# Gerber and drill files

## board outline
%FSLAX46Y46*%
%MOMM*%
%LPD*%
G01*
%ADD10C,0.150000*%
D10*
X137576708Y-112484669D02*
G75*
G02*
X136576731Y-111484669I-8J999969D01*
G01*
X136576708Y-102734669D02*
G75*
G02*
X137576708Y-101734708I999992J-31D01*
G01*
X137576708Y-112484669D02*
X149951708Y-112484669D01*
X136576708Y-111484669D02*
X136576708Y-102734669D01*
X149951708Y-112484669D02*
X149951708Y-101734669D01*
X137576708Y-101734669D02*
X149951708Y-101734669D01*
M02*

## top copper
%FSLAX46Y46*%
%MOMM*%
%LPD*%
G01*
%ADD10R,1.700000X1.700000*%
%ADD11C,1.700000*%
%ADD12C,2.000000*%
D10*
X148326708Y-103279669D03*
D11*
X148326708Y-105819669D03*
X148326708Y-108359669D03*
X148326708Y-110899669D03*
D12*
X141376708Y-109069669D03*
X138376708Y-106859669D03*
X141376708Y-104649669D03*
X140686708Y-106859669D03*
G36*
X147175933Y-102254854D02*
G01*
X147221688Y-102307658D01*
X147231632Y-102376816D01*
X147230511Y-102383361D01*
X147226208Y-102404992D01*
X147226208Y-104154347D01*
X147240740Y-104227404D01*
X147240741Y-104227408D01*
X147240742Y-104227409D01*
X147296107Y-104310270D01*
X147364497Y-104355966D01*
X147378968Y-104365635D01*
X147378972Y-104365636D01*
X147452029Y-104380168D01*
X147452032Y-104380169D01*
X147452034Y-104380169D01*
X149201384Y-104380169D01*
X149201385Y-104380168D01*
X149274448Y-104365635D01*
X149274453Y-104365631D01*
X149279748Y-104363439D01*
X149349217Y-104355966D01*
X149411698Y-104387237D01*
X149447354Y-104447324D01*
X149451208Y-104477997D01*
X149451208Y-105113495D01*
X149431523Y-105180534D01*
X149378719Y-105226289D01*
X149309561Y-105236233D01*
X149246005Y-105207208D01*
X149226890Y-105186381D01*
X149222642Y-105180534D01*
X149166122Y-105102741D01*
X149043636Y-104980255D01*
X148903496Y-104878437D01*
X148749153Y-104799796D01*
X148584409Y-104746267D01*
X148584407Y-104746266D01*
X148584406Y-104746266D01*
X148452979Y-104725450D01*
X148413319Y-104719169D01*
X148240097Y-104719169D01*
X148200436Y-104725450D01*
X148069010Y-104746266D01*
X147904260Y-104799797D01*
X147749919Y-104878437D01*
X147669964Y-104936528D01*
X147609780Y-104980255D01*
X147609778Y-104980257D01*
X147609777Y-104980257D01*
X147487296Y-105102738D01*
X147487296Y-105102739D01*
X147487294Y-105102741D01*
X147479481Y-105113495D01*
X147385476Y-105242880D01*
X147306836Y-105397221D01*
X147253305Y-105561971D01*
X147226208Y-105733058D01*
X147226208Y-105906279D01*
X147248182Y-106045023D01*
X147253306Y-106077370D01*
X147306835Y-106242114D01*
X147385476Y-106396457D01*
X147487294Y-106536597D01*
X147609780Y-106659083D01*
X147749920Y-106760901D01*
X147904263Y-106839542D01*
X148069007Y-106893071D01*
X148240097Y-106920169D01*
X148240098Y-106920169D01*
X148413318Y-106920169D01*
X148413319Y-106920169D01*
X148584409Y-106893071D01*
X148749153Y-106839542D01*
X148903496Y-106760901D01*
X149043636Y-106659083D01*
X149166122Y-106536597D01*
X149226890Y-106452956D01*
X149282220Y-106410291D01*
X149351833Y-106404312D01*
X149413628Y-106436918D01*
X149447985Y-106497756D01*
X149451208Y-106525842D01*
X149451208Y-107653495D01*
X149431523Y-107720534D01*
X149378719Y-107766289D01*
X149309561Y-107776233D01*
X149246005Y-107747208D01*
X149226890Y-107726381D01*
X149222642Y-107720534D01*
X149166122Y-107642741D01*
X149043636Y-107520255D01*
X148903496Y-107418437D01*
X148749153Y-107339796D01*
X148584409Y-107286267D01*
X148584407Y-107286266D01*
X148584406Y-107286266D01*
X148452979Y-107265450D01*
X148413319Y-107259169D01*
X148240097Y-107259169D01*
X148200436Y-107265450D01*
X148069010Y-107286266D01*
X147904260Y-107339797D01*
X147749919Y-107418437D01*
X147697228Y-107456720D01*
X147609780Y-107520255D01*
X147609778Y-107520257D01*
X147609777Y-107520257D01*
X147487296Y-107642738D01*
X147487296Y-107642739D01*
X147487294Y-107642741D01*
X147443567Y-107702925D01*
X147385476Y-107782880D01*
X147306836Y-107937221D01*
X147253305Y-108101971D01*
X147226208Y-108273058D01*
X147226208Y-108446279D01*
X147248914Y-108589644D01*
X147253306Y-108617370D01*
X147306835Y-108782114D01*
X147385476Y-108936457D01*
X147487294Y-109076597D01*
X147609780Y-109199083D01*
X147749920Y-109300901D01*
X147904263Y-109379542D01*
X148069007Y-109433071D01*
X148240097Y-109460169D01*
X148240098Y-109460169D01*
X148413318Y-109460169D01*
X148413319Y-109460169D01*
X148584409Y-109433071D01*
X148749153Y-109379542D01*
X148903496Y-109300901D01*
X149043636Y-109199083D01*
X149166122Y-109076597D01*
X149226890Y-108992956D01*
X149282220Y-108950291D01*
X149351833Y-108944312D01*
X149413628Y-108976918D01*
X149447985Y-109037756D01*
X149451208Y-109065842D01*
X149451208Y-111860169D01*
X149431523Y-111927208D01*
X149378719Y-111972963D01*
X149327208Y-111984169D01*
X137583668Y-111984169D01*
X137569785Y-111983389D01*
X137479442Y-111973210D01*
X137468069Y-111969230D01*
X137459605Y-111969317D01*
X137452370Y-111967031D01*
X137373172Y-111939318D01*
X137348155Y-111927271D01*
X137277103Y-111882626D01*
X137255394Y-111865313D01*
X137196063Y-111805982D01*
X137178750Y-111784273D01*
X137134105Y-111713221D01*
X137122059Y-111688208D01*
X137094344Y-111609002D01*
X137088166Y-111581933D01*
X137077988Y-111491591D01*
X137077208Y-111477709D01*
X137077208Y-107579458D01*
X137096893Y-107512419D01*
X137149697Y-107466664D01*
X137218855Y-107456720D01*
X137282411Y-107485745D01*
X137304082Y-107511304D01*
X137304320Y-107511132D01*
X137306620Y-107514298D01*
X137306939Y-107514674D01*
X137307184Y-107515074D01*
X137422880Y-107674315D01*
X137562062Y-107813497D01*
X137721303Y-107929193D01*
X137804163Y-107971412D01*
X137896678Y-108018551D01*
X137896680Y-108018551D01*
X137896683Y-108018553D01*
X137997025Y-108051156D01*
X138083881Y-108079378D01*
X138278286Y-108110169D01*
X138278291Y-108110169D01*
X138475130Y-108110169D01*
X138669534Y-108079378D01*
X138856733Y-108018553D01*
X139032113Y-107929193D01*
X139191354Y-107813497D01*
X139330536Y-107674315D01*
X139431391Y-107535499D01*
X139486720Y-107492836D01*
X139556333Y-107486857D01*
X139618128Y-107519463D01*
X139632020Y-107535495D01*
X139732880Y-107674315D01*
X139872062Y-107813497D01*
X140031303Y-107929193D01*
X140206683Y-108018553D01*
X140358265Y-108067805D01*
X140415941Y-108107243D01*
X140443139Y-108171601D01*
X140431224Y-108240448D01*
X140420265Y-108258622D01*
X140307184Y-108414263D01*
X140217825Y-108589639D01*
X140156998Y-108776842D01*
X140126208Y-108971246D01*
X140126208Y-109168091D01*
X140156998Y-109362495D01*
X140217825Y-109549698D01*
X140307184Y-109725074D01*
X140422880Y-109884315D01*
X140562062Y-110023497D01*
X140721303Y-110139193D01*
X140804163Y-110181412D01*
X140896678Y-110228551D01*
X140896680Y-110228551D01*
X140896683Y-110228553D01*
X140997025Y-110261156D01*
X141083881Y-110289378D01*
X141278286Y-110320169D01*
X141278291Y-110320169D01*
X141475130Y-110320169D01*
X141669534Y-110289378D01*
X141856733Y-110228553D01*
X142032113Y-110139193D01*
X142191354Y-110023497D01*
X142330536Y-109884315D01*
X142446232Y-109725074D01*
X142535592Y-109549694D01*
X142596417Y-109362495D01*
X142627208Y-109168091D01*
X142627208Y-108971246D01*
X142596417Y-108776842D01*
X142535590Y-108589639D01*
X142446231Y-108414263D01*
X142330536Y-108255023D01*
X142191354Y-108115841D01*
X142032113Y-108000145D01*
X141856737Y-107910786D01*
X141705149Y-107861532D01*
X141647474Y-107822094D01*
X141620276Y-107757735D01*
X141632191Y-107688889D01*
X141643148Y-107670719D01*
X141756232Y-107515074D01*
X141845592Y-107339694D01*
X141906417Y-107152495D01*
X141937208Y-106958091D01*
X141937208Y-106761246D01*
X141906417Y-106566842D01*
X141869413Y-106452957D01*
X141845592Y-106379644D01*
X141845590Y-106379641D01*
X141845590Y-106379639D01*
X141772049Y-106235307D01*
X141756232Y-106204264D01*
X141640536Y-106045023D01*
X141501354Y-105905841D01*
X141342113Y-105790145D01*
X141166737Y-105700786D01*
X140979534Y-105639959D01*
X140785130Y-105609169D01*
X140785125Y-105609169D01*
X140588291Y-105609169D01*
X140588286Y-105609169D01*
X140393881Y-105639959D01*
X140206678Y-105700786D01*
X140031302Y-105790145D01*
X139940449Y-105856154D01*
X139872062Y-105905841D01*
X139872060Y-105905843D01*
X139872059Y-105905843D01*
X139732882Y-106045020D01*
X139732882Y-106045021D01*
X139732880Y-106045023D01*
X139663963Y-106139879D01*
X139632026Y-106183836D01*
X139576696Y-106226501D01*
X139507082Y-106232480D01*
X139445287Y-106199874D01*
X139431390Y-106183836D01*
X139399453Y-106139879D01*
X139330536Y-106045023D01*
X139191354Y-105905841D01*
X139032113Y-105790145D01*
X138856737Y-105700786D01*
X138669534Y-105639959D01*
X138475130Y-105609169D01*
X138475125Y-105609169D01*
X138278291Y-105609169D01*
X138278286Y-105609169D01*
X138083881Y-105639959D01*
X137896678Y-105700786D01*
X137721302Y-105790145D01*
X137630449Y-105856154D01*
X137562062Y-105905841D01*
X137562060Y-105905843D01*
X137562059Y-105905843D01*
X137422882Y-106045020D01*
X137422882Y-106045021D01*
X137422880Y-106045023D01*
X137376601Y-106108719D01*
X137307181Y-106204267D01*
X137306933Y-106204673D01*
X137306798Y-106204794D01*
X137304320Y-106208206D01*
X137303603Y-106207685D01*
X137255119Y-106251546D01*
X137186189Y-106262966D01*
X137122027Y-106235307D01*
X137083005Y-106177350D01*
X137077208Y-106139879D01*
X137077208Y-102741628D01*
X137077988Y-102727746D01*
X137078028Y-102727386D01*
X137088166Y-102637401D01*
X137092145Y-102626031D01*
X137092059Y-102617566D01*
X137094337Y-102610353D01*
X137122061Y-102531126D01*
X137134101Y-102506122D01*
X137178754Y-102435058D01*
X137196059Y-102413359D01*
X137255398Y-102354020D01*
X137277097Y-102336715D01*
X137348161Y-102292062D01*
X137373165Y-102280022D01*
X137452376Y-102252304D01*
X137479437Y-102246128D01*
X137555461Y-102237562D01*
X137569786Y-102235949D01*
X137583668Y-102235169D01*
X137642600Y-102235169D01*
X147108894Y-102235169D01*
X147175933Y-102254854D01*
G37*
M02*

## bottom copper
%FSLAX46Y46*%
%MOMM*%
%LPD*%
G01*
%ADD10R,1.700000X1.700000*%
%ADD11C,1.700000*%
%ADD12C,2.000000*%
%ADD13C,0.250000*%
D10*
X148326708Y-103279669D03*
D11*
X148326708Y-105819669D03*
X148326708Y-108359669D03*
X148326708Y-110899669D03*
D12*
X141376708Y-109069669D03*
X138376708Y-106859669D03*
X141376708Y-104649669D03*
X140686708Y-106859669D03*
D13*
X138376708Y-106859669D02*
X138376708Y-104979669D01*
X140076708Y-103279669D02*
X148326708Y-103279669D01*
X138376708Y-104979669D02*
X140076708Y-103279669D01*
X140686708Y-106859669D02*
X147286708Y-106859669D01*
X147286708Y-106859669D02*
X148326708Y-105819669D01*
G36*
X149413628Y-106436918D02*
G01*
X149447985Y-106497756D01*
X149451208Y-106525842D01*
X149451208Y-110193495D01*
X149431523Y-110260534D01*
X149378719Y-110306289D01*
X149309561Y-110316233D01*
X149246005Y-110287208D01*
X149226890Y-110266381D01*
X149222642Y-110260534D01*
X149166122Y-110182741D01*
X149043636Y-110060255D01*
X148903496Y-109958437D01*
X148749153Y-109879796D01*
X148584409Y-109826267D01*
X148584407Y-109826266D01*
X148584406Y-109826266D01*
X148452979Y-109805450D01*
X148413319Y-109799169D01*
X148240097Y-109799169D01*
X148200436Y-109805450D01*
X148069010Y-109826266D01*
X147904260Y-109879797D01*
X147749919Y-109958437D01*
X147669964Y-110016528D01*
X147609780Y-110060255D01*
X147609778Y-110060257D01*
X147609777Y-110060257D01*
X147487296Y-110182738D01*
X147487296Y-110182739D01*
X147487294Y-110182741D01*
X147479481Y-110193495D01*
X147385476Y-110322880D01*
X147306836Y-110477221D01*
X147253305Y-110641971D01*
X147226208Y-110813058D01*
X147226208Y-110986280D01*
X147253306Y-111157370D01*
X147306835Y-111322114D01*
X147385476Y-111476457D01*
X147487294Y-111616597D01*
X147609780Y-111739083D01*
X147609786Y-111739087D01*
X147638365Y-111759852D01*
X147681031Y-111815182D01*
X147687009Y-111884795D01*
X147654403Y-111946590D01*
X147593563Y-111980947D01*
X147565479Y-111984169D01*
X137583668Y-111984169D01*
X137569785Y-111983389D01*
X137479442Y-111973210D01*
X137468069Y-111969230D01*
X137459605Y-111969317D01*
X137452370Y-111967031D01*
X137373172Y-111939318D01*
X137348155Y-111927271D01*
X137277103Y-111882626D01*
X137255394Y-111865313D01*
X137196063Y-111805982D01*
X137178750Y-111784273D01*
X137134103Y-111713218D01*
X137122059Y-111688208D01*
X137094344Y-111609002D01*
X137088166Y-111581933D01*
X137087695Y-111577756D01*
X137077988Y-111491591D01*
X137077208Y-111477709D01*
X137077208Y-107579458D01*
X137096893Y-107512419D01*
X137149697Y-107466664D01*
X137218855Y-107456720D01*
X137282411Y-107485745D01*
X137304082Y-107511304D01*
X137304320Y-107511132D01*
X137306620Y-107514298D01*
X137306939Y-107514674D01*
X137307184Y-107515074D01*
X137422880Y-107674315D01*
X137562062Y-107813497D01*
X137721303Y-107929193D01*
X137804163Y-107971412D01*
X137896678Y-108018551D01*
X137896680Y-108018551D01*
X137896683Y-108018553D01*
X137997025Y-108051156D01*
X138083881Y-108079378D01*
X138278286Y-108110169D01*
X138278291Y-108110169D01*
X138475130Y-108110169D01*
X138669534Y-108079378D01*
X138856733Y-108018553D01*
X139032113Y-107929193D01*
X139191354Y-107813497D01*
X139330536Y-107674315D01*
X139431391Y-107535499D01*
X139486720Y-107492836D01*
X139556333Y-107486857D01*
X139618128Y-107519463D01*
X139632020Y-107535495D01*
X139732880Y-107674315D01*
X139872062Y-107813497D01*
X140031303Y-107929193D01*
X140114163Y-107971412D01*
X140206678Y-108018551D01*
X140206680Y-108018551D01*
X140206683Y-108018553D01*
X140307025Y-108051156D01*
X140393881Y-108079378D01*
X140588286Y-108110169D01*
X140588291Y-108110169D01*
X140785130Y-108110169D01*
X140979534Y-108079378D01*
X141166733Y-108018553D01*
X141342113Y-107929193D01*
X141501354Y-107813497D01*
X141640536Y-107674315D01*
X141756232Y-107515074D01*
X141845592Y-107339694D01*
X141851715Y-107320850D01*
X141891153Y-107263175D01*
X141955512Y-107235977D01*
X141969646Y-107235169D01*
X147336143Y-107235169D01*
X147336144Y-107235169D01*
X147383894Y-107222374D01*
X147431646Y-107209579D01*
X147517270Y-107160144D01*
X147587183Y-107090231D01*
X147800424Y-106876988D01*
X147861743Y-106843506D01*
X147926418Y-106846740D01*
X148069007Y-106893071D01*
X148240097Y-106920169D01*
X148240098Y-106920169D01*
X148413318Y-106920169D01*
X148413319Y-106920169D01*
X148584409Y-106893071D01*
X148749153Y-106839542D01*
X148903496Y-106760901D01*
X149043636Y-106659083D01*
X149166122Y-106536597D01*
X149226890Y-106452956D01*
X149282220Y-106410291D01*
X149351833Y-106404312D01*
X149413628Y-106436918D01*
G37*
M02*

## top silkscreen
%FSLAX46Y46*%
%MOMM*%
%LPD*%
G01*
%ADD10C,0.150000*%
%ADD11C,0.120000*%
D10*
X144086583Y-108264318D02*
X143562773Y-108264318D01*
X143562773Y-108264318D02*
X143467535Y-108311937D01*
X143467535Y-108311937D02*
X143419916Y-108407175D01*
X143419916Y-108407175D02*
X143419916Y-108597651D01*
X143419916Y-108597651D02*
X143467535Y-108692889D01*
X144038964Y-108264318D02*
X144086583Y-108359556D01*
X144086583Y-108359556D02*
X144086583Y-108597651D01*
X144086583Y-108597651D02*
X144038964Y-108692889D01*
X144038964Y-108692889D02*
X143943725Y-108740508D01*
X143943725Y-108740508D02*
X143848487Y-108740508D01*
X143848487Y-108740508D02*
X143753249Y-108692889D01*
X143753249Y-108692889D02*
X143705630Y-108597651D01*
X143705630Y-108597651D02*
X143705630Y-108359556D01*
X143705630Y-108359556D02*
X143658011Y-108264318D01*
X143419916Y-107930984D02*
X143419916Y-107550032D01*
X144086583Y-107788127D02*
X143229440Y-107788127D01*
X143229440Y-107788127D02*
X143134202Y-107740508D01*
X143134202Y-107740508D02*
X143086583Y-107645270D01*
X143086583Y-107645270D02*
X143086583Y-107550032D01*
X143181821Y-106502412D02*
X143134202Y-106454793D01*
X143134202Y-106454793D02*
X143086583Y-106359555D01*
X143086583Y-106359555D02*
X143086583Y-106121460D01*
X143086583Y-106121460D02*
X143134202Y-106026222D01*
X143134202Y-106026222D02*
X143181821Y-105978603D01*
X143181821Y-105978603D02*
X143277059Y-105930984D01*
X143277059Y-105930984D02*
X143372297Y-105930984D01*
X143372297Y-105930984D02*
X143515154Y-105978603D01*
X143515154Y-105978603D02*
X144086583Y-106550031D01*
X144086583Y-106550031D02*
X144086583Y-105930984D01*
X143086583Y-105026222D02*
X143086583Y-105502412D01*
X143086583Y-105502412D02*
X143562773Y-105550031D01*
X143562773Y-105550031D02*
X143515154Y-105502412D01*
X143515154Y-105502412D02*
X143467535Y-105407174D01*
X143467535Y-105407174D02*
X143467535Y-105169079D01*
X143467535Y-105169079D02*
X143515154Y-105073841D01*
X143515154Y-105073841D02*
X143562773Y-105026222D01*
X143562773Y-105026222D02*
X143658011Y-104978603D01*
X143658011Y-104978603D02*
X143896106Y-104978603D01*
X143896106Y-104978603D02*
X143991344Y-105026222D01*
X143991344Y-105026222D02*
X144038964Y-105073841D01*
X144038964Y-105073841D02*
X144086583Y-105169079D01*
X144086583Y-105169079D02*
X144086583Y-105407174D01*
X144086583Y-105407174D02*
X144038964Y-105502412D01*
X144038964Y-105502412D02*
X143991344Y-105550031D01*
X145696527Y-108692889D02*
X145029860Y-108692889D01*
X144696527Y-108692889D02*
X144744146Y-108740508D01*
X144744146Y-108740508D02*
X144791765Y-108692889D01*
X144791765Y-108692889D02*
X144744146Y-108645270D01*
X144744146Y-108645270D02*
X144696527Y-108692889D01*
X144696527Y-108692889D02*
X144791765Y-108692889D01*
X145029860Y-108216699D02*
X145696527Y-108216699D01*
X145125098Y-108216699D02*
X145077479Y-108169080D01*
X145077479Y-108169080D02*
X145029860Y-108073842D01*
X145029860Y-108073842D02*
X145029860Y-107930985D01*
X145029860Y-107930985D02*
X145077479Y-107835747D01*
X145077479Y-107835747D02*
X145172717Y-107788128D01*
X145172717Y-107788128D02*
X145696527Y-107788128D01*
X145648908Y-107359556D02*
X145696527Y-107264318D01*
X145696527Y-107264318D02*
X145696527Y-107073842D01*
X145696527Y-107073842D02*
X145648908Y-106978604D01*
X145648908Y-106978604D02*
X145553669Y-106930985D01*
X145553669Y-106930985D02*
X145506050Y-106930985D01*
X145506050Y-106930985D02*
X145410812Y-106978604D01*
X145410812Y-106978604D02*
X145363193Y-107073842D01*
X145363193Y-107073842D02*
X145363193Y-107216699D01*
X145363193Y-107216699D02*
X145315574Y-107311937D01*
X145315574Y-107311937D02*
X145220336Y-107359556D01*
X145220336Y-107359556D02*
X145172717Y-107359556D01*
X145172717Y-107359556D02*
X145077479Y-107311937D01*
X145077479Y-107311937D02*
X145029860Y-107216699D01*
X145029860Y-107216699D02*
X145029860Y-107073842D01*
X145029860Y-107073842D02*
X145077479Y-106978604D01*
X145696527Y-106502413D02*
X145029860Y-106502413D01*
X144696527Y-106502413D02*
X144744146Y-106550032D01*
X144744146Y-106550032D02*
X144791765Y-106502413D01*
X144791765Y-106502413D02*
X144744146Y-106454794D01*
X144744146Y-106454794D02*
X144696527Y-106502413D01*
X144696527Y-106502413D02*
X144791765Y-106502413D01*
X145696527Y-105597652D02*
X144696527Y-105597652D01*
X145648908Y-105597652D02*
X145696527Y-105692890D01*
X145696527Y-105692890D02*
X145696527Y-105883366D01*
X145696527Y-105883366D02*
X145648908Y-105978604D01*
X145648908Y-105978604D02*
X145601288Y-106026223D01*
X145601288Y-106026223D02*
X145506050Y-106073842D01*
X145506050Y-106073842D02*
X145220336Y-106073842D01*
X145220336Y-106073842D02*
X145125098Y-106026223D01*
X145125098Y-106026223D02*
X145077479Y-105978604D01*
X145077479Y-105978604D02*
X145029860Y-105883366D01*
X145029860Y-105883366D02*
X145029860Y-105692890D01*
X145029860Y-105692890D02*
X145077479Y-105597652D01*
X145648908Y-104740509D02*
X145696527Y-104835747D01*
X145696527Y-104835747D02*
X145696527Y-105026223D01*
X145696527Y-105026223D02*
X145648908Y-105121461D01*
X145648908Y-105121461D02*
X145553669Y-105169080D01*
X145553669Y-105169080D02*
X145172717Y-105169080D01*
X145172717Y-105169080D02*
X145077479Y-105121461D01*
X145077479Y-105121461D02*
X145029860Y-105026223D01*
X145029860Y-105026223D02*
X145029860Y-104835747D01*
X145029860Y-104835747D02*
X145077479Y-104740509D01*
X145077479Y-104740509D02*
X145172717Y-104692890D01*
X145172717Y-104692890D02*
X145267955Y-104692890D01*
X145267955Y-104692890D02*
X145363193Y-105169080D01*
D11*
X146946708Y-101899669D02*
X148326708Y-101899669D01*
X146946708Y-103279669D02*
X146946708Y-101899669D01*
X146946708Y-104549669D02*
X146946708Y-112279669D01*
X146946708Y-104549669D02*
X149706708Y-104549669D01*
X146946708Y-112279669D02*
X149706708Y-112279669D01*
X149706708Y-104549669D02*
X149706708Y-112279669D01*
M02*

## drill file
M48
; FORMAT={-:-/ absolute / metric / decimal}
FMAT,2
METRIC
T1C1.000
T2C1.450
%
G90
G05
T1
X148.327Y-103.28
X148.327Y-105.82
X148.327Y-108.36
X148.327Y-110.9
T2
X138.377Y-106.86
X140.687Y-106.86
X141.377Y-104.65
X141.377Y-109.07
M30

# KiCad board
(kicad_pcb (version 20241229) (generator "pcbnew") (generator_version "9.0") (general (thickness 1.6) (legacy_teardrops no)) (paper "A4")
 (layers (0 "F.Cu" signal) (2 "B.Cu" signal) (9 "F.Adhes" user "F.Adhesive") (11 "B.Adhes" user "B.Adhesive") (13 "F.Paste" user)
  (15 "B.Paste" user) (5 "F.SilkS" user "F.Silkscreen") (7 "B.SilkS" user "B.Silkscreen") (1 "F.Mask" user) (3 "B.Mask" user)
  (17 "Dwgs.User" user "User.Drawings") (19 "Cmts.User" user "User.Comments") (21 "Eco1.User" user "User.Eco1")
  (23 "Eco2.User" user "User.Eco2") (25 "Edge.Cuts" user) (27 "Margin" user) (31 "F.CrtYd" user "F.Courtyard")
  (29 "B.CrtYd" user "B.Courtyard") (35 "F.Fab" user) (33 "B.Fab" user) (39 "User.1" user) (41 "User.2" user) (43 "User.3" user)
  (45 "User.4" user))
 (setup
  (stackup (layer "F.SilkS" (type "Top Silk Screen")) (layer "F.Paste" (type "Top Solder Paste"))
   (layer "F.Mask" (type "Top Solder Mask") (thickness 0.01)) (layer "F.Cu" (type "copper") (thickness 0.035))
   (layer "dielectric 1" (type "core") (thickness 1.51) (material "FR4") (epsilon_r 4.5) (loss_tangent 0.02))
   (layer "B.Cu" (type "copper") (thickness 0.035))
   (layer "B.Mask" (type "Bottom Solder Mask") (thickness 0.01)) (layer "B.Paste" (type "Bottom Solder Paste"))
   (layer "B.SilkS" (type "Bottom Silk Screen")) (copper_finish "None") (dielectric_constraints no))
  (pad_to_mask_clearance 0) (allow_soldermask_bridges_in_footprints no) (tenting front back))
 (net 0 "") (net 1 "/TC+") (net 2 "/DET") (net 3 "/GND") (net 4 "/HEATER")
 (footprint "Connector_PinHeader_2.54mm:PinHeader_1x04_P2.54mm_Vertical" (layer "F.Cu") (at 148.326708 103.279669)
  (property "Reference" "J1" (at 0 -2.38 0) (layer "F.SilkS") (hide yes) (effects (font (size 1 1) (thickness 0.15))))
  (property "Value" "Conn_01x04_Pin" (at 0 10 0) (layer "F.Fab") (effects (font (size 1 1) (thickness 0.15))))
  (fp_line (start -1.38 -1.38) (end 0 -1.38) (stroke (width 0.12) (type solid)) (layer "F.SilkS"))
  (fp_line (start -1.38 0) (end -1.38 -1.38) (stroke (width 0.12) (type solid)) (layer "F.SilkS"))
  (fp_line (start -1.38 1.27) (end -1.38 9) (stroke (width 0.12) (type solid)) (layer "F.SilkS"))
  (fp_line (start -1.38 1.27) (end 1.38 1.27) (stroke (width 0.12) (type solid)) (layer "F.SilkS"))
  (fp_line (start -1.38 9) (end 1.38 9) (stroke (width 0.12) (type solid)) (layer "F.SilkS"))
  (fp_line (start 1.38 1.27) (end 1.38 9) (stroke (width 0.12) (type solid)) (layer "F.SilkS"))
  (pad "1" thru_hole rect (at 0 0) (size 1.7 1.7) (drill 1) (layers "*.Cu" "*.Mask") (remove_unused_layers no) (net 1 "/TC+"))
  (pad "2" thru_hole circle (at 0 2.54) (size 1.7 1.7) (drill 1) (layers "*.Cu" "*.Mask") (remove_unused_layers no) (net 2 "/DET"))
  (pad "3" thru_hole circle (at 0 5.08) (size 1.7 1.7) (drill 1) (layers "*.Cu" "*.Mask") (remove_unused_layers no) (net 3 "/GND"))
  (pad "4" thru_hole circle (at 0 7.62) (size 1.7 1.7) (drill 1) (layers "*.Cu" "*.Mask") (remove_unused_layers no) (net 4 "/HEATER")))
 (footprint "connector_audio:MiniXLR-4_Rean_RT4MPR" (layer "B.Cu") (at 140.686708 106.859669 90)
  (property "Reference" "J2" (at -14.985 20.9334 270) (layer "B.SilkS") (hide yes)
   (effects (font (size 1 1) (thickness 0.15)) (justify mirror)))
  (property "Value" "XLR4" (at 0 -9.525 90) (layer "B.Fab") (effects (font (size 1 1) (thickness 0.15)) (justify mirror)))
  (pad "1" thru_hole circle (at -2.21 0.69 270) (size 2 2) (drill 1.45) (layers "*.Cu" "*.Mask") (remove_unused_layers no) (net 3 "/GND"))
  (pad "2" thru_hole circle (at 0 -2.31 270) (size 2 2) (drill 1.45) (layers "*.Cu" "*.Mask") (remove_unused_layers no) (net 1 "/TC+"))
  (pad "3" thru_hole circle (at 2.21 0.69 270) (size 2 2) (drill 1.45) (layers "*.Cu" "*.Mask") (remove_unused_layers no) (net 4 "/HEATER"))
  (pad "4" thru_hole circle (at 0 0 270) (size 2 2) (drill 1.45) (layers "*.Cu" "*.Mask") (remove_unused_layers no) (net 2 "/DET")))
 (gr_arc (start 137.576708 112.484669) (mid 136.869601 112.191776) (end 136.576708 111.484669) (stroke (width 0.15) (type default))
  (layer "Edge.Cuts"))
 (gr_arc (start 136.576708 102.734669) (mid 136.869601 102.027562) (end 137.576708 101.734669) (stroke (width 0.15) (type default))
  (layer "Edge.Cuts"))
 (gr_line (start 137.576708 112.484669) (end 149.951708 112.484669) (stroke (width 0.15) (type default)) (layer "Edge.Cuts"))
 (gr_line (start 136.576708 111.484669) (end 136.576708 102.734669) (stroke (width 0.15) (type default)) (layer "Edge.Cuts"))
 (gr_line (start 149.951708 112.484669) (end 149.951708 101.734669) (stroke (width 0.15) (type default)) (layer "Edge.Cuts"))
 (gr_line (start 137.576708 101.734669) (end 149.951708 101.734669) (stroke (width 0.15) (type default)) (layer "Edge.Cuts"))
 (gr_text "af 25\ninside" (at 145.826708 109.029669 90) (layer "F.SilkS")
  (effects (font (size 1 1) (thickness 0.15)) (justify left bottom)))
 (segment (start 138.376708 106.859669) (end 138.376708 104.979669) (width 0.25) (layer "B.Cu") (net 1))
 (segment (start 140.076708 103.279669) (end 148.326708 103.279669) (width 0.25) (layer "B.Cu") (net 1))
 (segment (start 138.376708 104.979669) (end 140.076708 103.279669) (width 0.25) (layer "B.Cu") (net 1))
 (segment (start 140.686708 106.859669) (end 147.286708 106.859669) (width 0.25) (layer "B.Cu") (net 2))
 (segment (start 147.286708 106.859669) (end 148.326708 105.819669) (width 0.25) (layer "B.Cu") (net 2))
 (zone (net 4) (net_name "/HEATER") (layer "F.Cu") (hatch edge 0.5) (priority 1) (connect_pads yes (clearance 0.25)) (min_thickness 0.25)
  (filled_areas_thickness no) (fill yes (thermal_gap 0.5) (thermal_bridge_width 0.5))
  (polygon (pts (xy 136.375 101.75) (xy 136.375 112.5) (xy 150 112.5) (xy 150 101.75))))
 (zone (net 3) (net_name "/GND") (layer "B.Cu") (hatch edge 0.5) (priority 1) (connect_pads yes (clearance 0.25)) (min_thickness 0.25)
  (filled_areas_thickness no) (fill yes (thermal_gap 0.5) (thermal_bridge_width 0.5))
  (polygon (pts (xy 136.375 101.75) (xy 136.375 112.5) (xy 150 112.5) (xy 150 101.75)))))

